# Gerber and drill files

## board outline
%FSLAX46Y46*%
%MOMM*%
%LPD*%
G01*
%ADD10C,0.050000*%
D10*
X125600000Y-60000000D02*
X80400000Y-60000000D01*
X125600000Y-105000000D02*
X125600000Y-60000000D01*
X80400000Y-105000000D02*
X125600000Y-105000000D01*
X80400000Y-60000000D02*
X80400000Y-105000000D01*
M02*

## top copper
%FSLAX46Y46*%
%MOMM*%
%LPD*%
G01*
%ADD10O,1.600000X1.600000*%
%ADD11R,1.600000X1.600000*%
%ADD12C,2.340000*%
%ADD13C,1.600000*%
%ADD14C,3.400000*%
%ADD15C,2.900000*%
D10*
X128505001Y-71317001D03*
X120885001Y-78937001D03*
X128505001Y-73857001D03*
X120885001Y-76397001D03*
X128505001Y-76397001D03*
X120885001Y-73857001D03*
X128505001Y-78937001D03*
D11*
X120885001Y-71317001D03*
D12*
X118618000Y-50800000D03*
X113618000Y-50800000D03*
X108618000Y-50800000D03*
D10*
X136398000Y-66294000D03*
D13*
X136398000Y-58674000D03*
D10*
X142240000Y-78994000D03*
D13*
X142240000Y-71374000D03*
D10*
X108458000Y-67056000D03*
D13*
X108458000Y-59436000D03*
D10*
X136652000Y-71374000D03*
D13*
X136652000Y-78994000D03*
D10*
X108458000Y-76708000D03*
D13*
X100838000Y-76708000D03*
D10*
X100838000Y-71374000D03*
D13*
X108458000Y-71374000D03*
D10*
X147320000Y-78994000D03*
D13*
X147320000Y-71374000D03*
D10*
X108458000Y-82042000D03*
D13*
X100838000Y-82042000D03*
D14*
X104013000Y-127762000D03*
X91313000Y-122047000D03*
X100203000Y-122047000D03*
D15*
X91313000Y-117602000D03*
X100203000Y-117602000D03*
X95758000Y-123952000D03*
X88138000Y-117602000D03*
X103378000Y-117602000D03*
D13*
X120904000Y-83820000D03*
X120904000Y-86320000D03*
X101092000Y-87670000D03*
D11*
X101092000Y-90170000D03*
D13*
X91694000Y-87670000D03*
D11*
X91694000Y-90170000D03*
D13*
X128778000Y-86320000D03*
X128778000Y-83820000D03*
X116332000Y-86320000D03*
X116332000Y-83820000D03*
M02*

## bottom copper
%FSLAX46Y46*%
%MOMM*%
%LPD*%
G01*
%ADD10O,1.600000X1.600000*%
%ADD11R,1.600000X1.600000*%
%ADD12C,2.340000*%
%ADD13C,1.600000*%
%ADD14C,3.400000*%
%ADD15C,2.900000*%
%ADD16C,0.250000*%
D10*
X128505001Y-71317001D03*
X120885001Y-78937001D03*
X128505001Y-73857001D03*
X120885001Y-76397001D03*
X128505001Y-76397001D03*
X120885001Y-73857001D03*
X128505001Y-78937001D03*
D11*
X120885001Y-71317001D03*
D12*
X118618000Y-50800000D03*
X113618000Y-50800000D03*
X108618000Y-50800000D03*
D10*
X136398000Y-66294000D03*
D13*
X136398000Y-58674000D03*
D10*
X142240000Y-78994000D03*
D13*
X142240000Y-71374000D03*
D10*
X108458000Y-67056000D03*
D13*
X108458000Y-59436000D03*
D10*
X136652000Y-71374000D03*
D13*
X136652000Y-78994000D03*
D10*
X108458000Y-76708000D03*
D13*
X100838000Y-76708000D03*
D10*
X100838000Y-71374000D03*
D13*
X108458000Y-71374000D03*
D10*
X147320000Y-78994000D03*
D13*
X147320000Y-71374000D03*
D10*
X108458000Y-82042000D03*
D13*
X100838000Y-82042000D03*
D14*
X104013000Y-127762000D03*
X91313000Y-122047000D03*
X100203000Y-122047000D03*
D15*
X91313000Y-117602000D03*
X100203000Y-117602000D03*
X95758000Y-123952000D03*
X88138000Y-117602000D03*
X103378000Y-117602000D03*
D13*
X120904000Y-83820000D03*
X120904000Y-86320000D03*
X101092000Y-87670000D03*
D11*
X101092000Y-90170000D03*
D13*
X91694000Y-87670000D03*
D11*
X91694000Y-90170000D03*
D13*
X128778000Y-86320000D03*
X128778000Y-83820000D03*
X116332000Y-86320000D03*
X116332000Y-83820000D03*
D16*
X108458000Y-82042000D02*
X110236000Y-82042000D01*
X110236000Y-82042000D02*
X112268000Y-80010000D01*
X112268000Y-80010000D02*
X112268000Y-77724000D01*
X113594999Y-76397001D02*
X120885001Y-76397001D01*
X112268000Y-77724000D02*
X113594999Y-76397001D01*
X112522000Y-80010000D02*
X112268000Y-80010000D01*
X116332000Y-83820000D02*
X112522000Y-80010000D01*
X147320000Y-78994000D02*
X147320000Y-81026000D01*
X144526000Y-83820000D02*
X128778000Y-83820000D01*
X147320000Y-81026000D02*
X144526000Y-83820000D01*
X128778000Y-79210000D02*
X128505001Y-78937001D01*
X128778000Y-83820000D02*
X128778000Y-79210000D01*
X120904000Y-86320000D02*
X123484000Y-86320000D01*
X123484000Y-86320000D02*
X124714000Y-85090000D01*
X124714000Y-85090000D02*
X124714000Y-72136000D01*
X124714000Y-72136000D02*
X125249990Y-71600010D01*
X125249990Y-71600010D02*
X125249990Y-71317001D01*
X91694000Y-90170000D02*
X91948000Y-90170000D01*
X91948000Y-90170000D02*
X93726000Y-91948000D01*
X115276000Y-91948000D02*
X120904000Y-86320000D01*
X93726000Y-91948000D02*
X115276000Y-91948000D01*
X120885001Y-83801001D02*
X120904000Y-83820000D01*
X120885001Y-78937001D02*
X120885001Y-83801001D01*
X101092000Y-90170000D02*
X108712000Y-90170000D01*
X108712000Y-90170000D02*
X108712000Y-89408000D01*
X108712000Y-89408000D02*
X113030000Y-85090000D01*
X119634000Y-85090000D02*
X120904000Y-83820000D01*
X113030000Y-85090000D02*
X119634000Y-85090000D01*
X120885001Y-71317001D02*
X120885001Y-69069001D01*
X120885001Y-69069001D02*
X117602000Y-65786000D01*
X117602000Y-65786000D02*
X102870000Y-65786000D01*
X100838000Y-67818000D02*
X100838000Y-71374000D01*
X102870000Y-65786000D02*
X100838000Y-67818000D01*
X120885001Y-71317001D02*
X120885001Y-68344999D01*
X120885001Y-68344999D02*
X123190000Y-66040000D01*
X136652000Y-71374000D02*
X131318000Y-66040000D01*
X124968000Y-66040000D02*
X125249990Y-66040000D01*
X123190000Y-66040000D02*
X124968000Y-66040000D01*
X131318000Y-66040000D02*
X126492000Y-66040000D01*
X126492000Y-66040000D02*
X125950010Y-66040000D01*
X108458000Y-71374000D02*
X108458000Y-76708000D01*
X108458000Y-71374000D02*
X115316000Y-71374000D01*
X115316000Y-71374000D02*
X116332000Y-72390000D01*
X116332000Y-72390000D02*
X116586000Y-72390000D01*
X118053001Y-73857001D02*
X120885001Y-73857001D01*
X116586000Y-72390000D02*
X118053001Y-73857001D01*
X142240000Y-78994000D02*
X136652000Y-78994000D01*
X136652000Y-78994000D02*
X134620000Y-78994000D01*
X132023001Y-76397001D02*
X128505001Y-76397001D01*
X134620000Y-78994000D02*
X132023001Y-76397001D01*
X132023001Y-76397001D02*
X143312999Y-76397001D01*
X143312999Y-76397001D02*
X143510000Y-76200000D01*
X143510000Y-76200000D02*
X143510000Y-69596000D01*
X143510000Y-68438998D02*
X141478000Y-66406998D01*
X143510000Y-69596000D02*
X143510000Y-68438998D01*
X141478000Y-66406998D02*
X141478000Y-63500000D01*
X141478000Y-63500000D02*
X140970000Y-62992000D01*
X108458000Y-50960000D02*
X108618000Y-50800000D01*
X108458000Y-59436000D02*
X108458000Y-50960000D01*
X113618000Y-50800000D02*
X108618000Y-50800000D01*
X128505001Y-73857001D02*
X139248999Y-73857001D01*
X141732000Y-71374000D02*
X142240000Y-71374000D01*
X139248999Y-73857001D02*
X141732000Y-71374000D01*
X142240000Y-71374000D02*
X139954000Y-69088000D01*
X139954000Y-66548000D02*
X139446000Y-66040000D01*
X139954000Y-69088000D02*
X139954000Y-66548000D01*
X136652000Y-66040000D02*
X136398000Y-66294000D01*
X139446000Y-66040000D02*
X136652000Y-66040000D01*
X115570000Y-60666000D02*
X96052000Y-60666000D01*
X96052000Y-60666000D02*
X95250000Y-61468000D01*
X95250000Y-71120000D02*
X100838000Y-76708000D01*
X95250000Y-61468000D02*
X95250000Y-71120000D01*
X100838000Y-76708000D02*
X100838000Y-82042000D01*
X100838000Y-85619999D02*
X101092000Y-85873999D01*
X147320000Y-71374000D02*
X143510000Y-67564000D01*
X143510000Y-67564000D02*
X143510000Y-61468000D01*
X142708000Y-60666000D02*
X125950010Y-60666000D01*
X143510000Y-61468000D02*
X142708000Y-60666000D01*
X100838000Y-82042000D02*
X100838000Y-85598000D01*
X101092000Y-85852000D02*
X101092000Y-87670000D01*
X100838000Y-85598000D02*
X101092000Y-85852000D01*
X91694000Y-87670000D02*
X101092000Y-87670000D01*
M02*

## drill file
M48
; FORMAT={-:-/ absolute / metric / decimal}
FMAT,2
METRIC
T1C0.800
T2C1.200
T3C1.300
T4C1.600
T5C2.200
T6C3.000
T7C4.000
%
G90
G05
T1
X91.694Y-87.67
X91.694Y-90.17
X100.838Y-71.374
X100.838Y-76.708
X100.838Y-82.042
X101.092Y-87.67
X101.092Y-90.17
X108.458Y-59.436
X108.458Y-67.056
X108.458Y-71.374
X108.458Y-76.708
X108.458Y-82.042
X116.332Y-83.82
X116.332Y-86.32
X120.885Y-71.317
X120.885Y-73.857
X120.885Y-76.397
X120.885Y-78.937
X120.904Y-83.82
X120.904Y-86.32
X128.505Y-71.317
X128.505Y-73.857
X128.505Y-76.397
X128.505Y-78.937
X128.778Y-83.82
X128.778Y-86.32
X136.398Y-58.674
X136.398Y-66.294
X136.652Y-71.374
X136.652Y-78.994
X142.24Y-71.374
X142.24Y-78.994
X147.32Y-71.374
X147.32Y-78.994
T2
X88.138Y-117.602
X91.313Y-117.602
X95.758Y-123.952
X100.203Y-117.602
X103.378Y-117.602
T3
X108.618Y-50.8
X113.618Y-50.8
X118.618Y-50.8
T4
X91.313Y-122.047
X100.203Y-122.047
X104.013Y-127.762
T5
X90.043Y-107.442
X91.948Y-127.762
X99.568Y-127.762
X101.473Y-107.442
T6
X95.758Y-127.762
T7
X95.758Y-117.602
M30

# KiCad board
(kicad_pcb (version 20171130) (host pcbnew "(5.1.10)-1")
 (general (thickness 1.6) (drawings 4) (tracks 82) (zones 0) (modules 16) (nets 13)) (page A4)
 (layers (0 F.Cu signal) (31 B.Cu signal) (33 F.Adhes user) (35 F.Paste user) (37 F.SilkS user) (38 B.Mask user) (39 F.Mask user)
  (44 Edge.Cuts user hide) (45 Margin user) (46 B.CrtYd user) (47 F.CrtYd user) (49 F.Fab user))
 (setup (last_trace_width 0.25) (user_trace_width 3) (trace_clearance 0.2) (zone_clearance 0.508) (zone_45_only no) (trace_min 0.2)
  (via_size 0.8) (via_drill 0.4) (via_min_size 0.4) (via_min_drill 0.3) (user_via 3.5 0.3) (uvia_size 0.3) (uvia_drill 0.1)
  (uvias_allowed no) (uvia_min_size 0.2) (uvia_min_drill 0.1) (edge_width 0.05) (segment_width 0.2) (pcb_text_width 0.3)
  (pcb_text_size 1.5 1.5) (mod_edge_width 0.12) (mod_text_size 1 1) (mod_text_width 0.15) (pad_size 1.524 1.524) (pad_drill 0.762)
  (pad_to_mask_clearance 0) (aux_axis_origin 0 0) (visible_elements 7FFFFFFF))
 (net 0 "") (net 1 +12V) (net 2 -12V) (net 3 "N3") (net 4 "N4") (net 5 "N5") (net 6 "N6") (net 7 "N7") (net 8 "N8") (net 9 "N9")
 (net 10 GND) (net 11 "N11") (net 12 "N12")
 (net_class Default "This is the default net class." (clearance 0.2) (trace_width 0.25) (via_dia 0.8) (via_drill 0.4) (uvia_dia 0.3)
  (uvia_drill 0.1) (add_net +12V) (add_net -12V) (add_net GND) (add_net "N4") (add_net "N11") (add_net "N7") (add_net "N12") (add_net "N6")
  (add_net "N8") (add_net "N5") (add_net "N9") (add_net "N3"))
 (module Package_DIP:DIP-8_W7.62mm (layer F.Cu) (at 120.885001 71.317001)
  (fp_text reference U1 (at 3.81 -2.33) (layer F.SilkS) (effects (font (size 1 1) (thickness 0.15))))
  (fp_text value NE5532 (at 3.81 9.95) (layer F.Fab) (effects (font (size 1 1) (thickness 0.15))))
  (pad 8 thru_hole oval (at 7.62 0) (size 1.6 1.6) (drill 0.8) (layers *.Cu *.Mask) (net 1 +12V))
  (pad 4 thru_hole oval (at 0 7.62) (size 1.6 1.6) (drill 0.8) (layers *.Cu *.Mask) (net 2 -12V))
  (pad 7 thru_hole oval (at 7.62 2.54) (size 1.6 1.6) (drill 0.8) (layers *.Cu *.Mask) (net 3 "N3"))
  (pad 3 thru_hole oval (at 0 5.08) (size 1.6 1.6) (drill 0.8) (layers *.Cu *.Mask) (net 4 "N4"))
  (pad 6 thru_hole oval (at 7.62 5.08) (size 1.6 1.6) (drill 0.8) (layers *.Cu *.Mask) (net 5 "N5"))
  (pad 2 thru_hole oval (at 0 2.54) (size 1.6 1.6) (drill 0.8) (layers *.Cu *.Mask) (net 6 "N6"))
  (pad 5 thru_hole oval (at 7.62 7.62) (size 1.6 1.6) (drill 0.8) (layers *.Cu *.Mask) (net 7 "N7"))
  (pad 1 thru_hole rect (at 0 0) (size 1.6 1.6) (drill 0.8) (layers *.Cu *.Mask) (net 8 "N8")))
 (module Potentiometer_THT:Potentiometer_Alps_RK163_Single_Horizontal (layer F.Cu) (at 118.618 50.8 90)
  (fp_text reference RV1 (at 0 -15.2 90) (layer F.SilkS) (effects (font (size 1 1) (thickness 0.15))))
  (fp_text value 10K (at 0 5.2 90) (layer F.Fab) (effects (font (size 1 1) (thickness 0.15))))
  (pad 1 thru_hole circle (at 0 0 90) (size 2.34 2.34) (drill 1.3) (layers *.Cu *.Mask) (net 5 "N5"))
  (pad 2 thru_hole circle (at 0 -5 90) (size 2.34 2.34) (drill 1.3) (layers *.Cu *.Mask) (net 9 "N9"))
  (pad 3 thru_hole circle (at 0 -10 90) (size 2.34 2.34) (drill 1.3) (layers *.Cu *.Mask) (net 9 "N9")))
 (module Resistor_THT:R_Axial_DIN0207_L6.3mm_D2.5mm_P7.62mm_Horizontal (layer F.Cu) (at 136.398 58.674 270)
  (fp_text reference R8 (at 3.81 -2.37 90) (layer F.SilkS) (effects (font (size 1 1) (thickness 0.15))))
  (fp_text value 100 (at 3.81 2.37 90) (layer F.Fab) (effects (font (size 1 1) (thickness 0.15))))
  (pad 2 thru_hole oval (at 7.62 0 270) (size 1.6 1.6) (drill 0.8) (layers *.Cu *.Mask) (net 3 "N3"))
  (pad 1 thru_hole circle (at 0 0 270) (size 1.6 1.6) (drill 0.8) (layers *.Cu *.Mask)))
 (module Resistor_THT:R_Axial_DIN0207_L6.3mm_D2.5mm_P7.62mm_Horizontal (layer F.Cu) (at 142.24 71.374 270)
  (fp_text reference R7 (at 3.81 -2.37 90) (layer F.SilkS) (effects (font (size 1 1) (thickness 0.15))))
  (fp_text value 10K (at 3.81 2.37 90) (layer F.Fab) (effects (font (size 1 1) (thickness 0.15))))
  (pad 2 thru_hole oval (at 7.62 0 270) (size 1.6 1.6) (drill 0.8) (layers *.Cu *.Mask) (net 5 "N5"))
  (pad 1 thru_hole circle (at 0 0 270) (size 1.6 1.6) (drill 0.8) (layers *.Cu *.Mask) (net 3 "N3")))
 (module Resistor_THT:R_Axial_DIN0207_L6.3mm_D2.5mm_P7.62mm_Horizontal (layer F.Cu) (at 108.458 59.436 270)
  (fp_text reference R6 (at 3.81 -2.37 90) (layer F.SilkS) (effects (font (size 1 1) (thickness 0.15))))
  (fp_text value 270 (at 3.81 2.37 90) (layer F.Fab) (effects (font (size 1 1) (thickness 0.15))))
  (pad 2 thru_hole oval (at 7.62 0 270) (size 1.6 1.6) (drill 0.8) (layers *.Cu *.Mask) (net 6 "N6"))
  (pad 1 thru_hole circle (at 0 0 270) (size 1.6 1.6) (drill 0.8) (layers *.Cu *.Mask) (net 9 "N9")))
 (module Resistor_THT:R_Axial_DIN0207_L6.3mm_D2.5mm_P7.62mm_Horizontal (layer F.Cu) (at 136.652 78.994 90)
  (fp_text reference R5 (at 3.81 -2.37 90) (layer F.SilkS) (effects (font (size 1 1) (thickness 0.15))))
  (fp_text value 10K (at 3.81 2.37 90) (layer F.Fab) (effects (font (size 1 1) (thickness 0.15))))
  (pad 2 thru_hole oval (at 7.62 0 90) (size 1.6 1.6) (drill 0.8) (layers *.Cu *.Mask) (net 8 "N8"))
  (pad 1 thru_hole circle (at 0 0 90) (size 1.6 1.6) (drill 0.8) (layers *.Cu *.Mask) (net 5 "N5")))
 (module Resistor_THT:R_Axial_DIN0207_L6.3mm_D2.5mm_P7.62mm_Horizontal (layer F.Cu) (at 100.838 76.708)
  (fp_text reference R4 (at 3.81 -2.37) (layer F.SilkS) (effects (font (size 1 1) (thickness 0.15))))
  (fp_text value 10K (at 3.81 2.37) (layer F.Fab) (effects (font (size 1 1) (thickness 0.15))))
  (pad 2 thru_hole oval (at 7.62 0) (size 1.6 1.6) (drill 0.8) (layers *.Cu *.Mask) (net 6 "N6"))
  (pad 1 thru_hole circle (at 0 0) (size 1.6 1.6) (drill 0.8) (layers *.Cu *.Mask) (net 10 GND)))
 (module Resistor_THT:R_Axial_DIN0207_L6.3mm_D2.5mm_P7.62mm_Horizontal (layer F.Cu) (at 108.458 71.374 180)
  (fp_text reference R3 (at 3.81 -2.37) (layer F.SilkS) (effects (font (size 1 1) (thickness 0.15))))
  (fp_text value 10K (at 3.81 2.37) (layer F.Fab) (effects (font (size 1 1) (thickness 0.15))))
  (pad 2 thru_hole oval (at 7.62 0 180) (size 1.6 1.6) (drill 0.8) (layers *.Cu *.Mask) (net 8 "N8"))
  (pad 1 thru_hole circle (at 0 0 180) (size 1.6 1.6) (drill 0.8) (layers *.Cu *.Mask) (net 6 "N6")))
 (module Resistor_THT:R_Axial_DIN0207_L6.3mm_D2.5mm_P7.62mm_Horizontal (layer F.Cu) (at 147.32 71.374 270)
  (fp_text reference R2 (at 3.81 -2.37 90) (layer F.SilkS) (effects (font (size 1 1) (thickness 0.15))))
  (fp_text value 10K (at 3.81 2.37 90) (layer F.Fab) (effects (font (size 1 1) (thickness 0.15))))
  (pad 2 thru_hole oval (at 7.62 0 270) (size 1.6 1.6) (drill 0.8) (layers *.Cu *.Mask) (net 7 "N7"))
  (pad 1 thru_hole circle (at 0 0 270) (size 1.6 1.6) (drill 0.8) (layers *.Cu *.Mask) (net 10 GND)))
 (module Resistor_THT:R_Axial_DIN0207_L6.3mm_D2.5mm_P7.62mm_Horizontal (layer F.Cu) (at 100.838 82.042)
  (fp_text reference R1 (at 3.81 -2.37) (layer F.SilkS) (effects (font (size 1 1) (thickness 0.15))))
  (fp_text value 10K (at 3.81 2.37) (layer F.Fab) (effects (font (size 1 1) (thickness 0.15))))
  (pad 2 thru_hole oval (at 7.62 0) (size 1.6 1.6) (drill 0.8) (layers *.Cu *.Mask) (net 4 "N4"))
  (pad 1 thru_hole circle (at 0 0) (size 1.6 1.6) (drill 0.8) (layers *.Cu *.Mask) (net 10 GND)))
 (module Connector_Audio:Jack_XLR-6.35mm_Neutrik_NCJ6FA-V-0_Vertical (layer F.Cu) (at 103.378 117.602)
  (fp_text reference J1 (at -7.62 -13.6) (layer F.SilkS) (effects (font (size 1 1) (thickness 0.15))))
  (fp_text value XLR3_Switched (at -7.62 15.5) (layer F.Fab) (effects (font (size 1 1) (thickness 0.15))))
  (pad "" np_thru_hole circle (at -1.905 -10.16) (size 2.2 2.2) (drill 2.2) (layers *.Cu *.Mask))
  (pad "" np_thru_hole circle (at -13.335 -10.16) (size 2.2 2.2) (drill 2.2) (layers *.Cu *.Mask))
  (pad G thru_hole circle (at 0.635 10.16) (size 3.4 3.4) (drill 1.6) (layers *.Cu *.Mask))
  (pad "" np_thru_hole circle (at -11.43 10.16) (size 2.2 2.2) (drill 2.2) (layers *.Cu *.Mask))
  (pad "" np_thru_hole circle (at -3.81 10.16) (size 2.2 2.2) (drill 2.2) (layers *.Cu *.Mask))
  (pad "" np_thru_hole circle (at -7.62 10.16) (size 3 3) (drill 3) (layers *.Cu *.Mask))
  (pad T thru_hole circle (at -12.065 4.445) (size 3.4 3.4) (drill 1.6) (layers *.Cu *.Mask))
  (pad T thru_hole circle (at -3.175 4.445) (size 3.4 3.4) (drill 1.6) (layers *.Cu *.Mask))
  (pad R thru_hole circle (at -12.065 0) (size 2.9 2.9) (drill 1.2) (layers *.Cu *.Mask))
  (pad S thru_hole circle (at -3.175 0) (size 2.9 2.9) (drill 1.2) (layers *.Cu *.Mask))
  (pad 3 thru_hole circle (at -7.62 6.35) (size 2.9 2.9) (drill 1.2) (layers *.Cu *.Mask) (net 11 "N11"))
  (pad 2 thru_hole circle (at -15.24 0) (size 2.9 2.9) (drill 1.2) (layers *.Cu *.Mask) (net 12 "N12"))
  (pad 1 thru_hole circle (at 0 0) (size 2.9 2.9) (drill 1.2) (layers *.Cu *.Mask))
  (pad "" np_thru_hole circle (at -7.62 0) (size 4 4) (drill 4) (layers *.Cu *.Mask)))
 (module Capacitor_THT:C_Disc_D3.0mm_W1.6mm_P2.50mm (layer F.Cu) (at 120.904 86.32 90)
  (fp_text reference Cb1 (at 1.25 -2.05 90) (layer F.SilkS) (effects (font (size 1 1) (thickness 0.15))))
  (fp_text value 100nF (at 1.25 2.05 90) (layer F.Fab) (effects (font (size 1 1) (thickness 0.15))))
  (pad 2 thru_hole circle (at 2.5 0 90) (size 1.6 1.6) (drill 0.8) (layers *.Cu *.Mask) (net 2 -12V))
  (pad 1 thru_hole circle (at 0 0 90) (size 1.6 1.6) (drill 0.8) (layers *.Cu *.Mask) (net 1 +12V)))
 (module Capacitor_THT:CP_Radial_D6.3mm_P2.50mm (layer F.Cu) (at 101.092 90.17 90)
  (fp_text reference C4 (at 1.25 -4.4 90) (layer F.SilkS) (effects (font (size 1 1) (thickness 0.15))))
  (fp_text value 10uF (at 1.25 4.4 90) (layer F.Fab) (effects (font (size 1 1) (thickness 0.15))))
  (pad 2 thru_hole circle (at 2.5 0 90) (size 1.6 1.6) (drill 0.8) (layers *.Cu *.Mask) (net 10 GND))
  (pad 1 thru_hole rect (at 0 0 90) (size 1.6 1.6) (drill 0.8) (layers *.Cu *.Mask) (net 2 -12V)))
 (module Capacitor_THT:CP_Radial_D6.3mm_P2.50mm (layer F.Cu) (at 91.694 90.17 90)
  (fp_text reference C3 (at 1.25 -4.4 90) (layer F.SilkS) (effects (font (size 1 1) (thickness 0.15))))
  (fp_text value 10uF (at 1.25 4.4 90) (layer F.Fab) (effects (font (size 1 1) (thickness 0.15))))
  (pad 2 thru_hole circle (at 2.5 0 90) (size 1.6 1.6) (drill 0.8) (layers *.Cu *.Mask) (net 10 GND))
  (pad 1 thru_hole rect (at 0 0 90) (size 1.6 1.6) (drill 0.8) (layers *.Cu *.Mask) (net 1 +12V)))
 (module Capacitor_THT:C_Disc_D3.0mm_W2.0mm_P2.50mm (layer F.Cu) (at 128.778 83.82 270)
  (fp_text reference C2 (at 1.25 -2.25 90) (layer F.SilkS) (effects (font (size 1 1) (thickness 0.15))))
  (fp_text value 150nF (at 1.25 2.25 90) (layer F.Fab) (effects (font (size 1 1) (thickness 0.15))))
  (pad 2 thru_hole circle (at 2.5 0 270) (size 1.6 1.6) (drill 0.8) (layers *.Cu *.Mask) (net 12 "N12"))
  (pad 1 thru_hole circle (at 0 0 270) (size 1.6 1.6) (drill 0.8) (layers *.Cu *.Mask) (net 7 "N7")))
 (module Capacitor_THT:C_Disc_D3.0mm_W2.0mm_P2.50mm (layer F.Cu) (at 116.332 83.82 270)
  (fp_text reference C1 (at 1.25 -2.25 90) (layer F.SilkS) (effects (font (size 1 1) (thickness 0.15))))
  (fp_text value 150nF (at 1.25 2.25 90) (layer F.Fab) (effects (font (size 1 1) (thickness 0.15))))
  (pad 2 thru_hole circle (at 2.5 0 270) (size 1.6 1.6) (drill 0.8) (layers *.Cu *.Mask) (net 11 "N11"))
  (pad 1 thru_hole circle (at 0 0 270) (size 1.6 1.6) (drill 0.8) (layers *.Cu *.Mask) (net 4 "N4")))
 (gr_line (start 125.6 60) (end 80.4 60) (layer Edge.Cuts) (width 0.05))
 (gr_line (start 125.6 105) (end 125.6 60) (layer Edge.Cuts) (width 0.05))
 (gr_line (start 80.4 105) (end 125.6 105) (layer Edge.Cuts) (width 0.05))
 (gr_line (start 80.4 60) (end 80.4 105) (layer Edge.Cuts) (width 0.05))
 (segment (start 108.458 82.042) (end 110.236 82.042) (width 0.25) (layer B.Cu) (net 4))
 (segment (start 110.236 82.042) (end 112.268 80.01) (width 0.25) (layer B.Cu) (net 4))
 (segment (start 112.268 80.01) (end 112.268 77.724) (width 0.25) (layer B.Cu) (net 4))
 (segment (start 113.594999 76.397001) (end 120.885001 76.397001) (width 0.25) (layer B.Cu) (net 4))
 (segment (start 112.268 77.724) (end 113.594999 76.397001) (width 0.25) (layer B.Cu) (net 4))
 (segment (start 112.522 80.01) (end 112.268 80.01) (width 0.25) (layer B.Cu) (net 4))
 (segment (start 116.332 83.82) (end 112.522 80.01) (width 0.25) (layer B.Cu) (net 4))
 (segment (start 147.32 78.994) (end 147.32 81.026) (width 0.25) (layer B.Cu) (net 7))
 (segment (start 144.526 83.82) (end 128.778 83.82) (width 0.25) (layer B.Cu) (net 7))
 (segment (start 147.32 81.026) (end 144.526 83.82) (width 0.25) (layer B.Cu) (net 7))
 (segment (start 128.778 79.21) (end 128.505001 78.937001) (width 0.25) (layer B.Cu) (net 7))
 (segment (start 128.778 83.82) (end 128.778 79.21) (width 0.25) (layer B.Cu) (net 7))
 (segment (start 120.904 86.32) (end 123.484 86.32) (width 0.25) (layer B.Cu) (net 1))
 (segment (start 123.484 86.32) (end 124.714 85.09) (width 0.25) (layer B.Cu) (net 1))
 (segment (start 124.714 85.09) (end 124.714 72.136) (width 0.25) (layer B.Cu) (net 1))
 (segment (start 124.714 72.136) (end 125.24999 71.60001) (width 0.25) (layer B.Cu) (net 1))
 (segment (start 125.24999 71.60001) (end 125.24999 71.317001) (width 0.25) (layer B.Cu) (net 1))
 (segment (start 91.694 90.17) (end 91.948 90.17) (width 0.25) (layer B.Cu) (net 1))
 (segment (start 91.948 90.17) (end 93.726 91.948) (width 0.25) (layer B.Cu) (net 1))
 (segment (start 115.276 91.948) (end 120.904 86.32) (width 0.25) (layer B.Cu) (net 1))
 (segment (start 93.726 91.948) (end 115.276 91.948) (width 0.25) (layer B.Cu) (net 1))
 (segment (start 120.885001 83.801001) (end 120.904 83.82) (width 0.25) (layer B.Cu) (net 2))
 (segment (start 120.885001 78.937001) (end 120.885001 83.801001) (width 0.25) (layer B.Cu) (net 2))
 (segment (start 101.092 90.17) (end 108.712 90.17) (width 0.25) (layer B.Cu) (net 2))
 (segment (start 108.712 90.17) (end 108.712 89.408) (width 0.25) (layer B.Cu) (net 2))
 (segment (start 108.712 89.408) (end 113.03 85.09) (width 0.25) (layer B.Cu) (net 2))
 (segment (start 119.634 85.09) (end 120.904 83.82) (width 0.25) (layer B.Cu) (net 2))
 (segment (start 113.03 85.09) (end 119.634 85.09) (width 0.25) (layer B.Cu) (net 2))
 (segment (start 120.885001 71.317001) (end 120.885001 69.069001) (width 0.25) (layer B.Cu) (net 8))
 (segment (start 120.885001 69.069001) (end 117.602 65.786) (width 0.25) (layer B.Cu) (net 8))
 (segment (start 117.602 65.786) (end 102.87 65.786) (width 0.25) (layer B.Cu) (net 8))
 (segment (start 100.838 67.818) (end 100.838 71.374) (width 0.25) (layer B.Cu) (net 8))
 (segment (start 102.87 65.786) (end 100.838 67.818) (width 0.25) (layer B.Cu) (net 8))
 (segment (start 120.885001 71.317001) (end 120.885001 68.344999) (width 0.25) (layer B.Cu) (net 8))
 (segment (start 120.885001 68.344999) (end 123.19 66.04) (width 0.25) (layer B.Cu) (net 8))
 (segment (start 136.652 71.374) (end 131.318 66.04) (width 0.25) (layer B.Cu) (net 8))
 (segment (start 124.968 66.04) (end 125.24999 66.04) (width 0.25) (layer B.Cu) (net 8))
 (segment (start 123.19 66.04) (end 124.968 66.04) (width 0.25) (layer B.Cu) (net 8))
 (segment (start 131.318 66.04) (end 126.492 66.04) (width 0.25) (layer B.Cu) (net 8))
 (segment (start 126.492 66.04) (end 125.95001 66.04) (width 0.25) (layer B.Cu) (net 8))
 (segment (start 108.458 71.374) (end 108.458 76.708) (width 0.25) (layer B.Cu) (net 6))
 (segment (start 108.458 71.374) (end 115.316 71.374) (width 0.25) (layer B.Cu) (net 6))
 (segment (start 115.316 71.374) (end 116.332 72.39) (width 0.25) (layer B.Cu) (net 6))
 (segment (start 116.332 72.39) (end 116.586 72.39) (width 0.25) (layer B.Cu) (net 6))
 (segment (start 118.053001 73.857001) (end 120.885001 73.857001) (width 0.25) (layer B.Cu) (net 6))
 (segment (start 116.586 72.39) (end 118.053001 73.857001) (width 0.25) (layer B.Cu) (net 6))
 (segment (start 142.24 78.994) (end 136.652 78.994) (width 0.25) (layer B.Cu) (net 5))
 (segment (start 136.652 78.994) (end 134.62 78.994) (width 0.25) (layer B.Cu) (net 5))
 (segment (start 132.023001 76.397001) (end 128.505001 76.397001) (width 0.25) (layer B.Cu) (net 5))
 (segment (start 134.62 78.994) (end 132.023001 76.397001) (width 0.25) (layer B.Cu) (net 5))
 (segment (start 132.023001 76.397001) (end 143.312999 76.397001) (width 0.25) (layer B.Cu) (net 5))
 (segment (start 143.312999 76.397001) (end 143.51 76.2) (width 0.25) (layer B.Cu) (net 5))
 (segment (start 143.51 76.2) (end 143.51 69.596) (width 0.25) (layer B.Cu) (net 5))
 (segment (start 143.51 68.438998) (end 141.478 66.406998) (width 0.25) (layer B.Cu) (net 5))
 (segment (start 143.51 69.596) (end 143.51 68.438998) (width 0.25) (layer B.Cu) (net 5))
 (segment (start 141.478 66.406998) (end 141.478 63.5) (width 0.25) (layer B.Cu) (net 5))
 (segment (start 141.478 63.5) (end 140.97 62.992) (width 0.25) (layer B.Cu) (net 5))
 (segment (start 108.458 50.96) (end 108.618 50.8) (width 0.25) (layer B.Cu) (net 9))
 (segment (start 108.458 59.436) (end 108.458 50.96) (width 0.25) (layer B.Cu) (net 9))
 (segment (start 113.618 50.8) (end 108.618 50.8) (width 0.25) (layer B.Cu) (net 9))
 (segment (start 128.505001 73.857001) (end 139.248999 73.857001) (width 0.25) (layer B.Cu) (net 3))
 (segment (start 141.732 71.374) (end 142.24 71.374) (width 0.25) (layer B.Cu) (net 3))
 (segment (start 139.248999 73.857001) (end 141.732 71.374) (width 0.25) (layer B.Cu) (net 3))
 (segment (start 142.24 71.374) (end 139.954 69.088) (width 0.25) (layer B.Cu) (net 3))
 (segment (start 139.954 66.548) (end 139.446 66.04) (width 0.25) (layer B.Cu) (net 3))
 (segment (start 139.954 69.088) (end 139.954 66.548) (width 0.25) (layer B.Cu) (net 3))
 (segment (start 136.652 66.04) (end 136.398 66.294) (width 0.25) (layer B.Cu) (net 3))
 (segment (start 139.446 66.04) (end 136.652 66.04) (width 0.25) (layer B.Cu) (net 3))
 (segment (start 115.57 60.666) (end 96.052 60.666) (width 0.25) (layer B.Cu) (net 10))
 (segment (start 96.052 60.666) (end 95.25 61.468) (width 0.25) (layer B.Cu) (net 10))
 (segment (start 95.25 71.12) (end 100.838 76.708) (width 0.25) (layer B.Cu) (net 10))
 (segment (start 95.25 61.468) (end 95.25 71.12) (width 0.25) (layer B.Cu) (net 10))
 (segment (start 100.838 76.708) (end 100.838 82.042) (width 0.25) (layer B.Cu) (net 10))
 (segment (start 100.838 85.619999) (end 101.092 85.873999) (width 0.25) (layer B.Cu) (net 10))
 (segment (start 147.32 71.374) (end 143.51 67.564) (width 0.25) (layer B.Cu) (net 10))
 (segment (start 143.51 67.564) (end 143.51 61.468) (width 0.25) (layer B.Cu) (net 10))
 (segment (start 142.708 60.666) (end 125.95001 60.666) (width 0.25) (layer B.Cu) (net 10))
 (segment (start 143.51 61.468) (end 142.708 60.666) (width 0.25) (layer B.Cu) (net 10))
 (segment (start 100.838 82.042) (end 100.838 85.598) (width 0.25) (layer B.Cu) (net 10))
 (segment (start 101.092 85.852) (end 101.092 87.67) (width 0.25) (layer B.Cu) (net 10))
 (segment (start 100.838 85.598) (end 101.092 85.852) (width 0.25) (layer B.Cu) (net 10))
 (segment (start 91.694 87.67) (end 101.092 87.67) (width 0.25) (layer B.Cu) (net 10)))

